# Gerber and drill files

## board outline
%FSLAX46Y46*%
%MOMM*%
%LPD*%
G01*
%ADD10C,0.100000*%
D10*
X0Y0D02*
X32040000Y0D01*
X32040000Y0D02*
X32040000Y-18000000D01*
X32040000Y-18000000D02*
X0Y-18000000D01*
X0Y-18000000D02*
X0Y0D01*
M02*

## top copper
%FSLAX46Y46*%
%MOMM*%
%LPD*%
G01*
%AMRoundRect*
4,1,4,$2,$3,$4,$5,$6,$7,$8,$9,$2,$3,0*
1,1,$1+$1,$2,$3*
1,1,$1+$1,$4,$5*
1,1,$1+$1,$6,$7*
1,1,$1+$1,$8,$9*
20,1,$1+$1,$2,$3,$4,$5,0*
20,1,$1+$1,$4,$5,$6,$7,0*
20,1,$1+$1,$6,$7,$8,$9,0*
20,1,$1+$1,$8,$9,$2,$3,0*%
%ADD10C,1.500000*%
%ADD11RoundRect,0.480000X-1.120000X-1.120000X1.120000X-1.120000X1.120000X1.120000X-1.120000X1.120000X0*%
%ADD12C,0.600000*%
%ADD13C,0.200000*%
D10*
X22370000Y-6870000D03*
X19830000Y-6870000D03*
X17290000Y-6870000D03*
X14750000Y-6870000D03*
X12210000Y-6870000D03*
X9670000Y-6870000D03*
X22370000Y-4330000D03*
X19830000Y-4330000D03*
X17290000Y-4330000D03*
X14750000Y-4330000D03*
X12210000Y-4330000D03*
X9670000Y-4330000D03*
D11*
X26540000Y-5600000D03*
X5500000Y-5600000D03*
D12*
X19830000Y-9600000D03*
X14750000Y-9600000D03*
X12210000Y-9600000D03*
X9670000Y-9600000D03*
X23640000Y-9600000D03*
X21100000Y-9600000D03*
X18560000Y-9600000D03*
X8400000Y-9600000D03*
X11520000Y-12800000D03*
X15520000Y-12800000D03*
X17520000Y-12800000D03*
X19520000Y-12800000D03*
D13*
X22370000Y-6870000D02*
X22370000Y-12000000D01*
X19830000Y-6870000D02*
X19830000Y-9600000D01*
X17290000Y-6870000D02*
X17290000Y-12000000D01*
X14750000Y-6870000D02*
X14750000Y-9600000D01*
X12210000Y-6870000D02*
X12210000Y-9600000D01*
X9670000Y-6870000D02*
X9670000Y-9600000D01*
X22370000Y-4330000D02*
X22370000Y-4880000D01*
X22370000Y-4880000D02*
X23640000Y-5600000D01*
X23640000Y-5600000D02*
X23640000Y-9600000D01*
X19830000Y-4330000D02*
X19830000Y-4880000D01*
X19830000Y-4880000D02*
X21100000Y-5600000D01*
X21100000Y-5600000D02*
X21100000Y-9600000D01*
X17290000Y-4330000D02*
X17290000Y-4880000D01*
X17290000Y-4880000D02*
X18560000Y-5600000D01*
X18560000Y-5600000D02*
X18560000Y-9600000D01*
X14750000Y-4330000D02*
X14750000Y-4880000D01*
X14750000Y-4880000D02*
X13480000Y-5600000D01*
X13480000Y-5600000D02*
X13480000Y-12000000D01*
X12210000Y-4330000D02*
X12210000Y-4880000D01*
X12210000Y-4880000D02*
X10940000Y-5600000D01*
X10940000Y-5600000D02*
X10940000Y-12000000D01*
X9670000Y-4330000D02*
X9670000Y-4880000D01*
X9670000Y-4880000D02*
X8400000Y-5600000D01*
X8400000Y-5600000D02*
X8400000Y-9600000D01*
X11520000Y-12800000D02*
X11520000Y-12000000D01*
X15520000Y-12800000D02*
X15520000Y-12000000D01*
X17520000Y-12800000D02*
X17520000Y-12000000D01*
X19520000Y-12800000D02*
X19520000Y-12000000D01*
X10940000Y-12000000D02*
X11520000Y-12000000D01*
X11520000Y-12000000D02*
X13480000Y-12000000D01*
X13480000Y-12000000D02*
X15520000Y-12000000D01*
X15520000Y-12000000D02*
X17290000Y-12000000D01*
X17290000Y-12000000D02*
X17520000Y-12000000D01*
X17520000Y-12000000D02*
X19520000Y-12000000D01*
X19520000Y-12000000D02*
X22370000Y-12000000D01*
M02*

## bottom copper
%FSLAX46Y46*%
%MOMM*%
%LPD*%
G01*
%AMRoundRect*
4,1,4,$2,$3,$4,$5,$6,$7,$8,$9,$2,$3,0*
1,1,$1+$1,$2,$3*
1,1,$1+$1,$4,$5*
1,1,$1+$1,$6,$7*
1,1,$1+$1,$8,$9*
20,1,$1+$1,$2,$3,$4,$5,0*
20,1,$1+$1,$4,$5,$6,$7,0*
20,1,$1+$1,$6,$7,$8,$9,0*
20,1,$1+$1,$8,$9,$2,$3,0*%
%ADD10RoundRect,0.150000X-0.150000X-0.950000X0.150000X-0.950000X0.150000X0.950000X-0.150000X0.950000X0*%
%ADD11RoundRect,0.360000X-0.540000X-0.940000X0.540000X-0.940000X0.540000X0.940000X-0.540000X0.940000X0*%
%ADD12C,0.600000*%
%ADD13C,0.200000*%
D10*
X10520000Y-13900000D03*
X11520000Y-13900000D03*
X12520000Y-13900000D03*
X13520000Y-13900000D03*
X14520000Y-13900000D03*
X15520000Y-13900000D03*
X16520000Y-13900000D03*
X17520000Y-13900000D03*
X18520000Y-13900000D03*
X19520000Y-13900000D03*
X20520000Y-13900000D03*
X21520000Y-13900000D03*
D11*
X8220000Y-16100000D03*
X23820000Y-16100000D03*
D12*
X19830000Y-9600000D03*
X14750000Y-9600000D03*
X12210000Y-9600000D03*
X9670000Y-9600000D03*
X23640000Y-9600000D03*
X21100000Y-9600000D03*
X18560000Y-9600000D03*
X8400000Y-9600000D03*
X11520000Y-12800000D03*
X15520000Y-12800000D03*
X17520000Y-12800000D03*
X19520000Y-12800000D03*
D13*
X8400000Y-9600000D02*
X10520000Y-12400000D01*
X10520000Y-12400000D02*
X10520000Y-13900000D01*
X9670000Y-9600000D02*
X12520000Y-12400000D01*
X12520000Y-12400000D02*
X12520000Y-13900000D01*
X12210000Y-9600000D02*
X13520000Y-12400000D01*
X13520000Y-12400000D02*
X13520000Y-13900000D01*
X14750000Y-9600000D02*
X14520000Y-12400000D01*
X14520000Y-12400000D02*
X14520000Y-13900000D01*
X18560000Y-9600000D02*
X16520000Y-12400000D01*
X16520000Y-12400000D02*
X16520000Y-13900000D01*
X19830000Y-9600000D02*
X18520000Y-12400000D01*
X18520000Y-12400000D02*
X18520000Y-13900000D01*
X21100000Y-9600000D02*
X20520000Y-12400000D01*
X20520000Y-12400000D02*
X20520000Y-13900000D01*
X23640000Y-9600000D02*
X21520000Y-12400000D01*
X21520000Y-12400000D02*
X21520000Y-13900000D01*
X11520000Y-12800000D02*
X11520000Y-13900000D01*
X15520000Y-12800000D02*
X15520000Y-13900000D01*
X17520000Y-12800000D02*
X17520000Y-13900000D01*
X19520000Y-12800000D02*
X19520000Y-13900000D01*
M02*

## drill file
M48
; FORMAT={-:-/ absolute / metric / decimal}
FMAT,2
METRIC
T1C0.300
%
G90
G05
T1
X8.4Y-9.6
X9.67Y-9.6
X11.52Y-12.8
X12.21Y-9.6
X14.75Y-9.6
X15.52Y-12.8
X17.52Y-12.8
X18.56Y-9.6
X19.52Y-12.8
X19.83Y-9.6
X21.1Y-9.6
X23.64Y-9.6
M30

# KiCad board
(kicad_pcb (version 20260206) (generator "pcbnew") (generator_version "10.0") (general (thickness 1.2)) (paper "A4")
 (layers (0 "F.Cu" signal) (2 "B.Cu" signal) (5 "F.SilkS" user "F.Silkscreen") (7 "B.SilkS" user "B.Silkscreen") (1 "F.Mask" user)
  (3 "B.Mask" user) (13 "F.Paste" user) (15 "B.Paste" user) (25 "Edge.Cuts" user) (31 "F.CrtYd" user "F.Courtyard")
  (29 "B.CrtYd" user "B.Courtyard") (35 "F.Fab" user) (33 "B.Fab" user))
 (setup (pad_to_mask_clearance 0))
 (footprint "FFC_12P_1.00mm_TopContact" (at 16.02 15) (layer "B.Cu")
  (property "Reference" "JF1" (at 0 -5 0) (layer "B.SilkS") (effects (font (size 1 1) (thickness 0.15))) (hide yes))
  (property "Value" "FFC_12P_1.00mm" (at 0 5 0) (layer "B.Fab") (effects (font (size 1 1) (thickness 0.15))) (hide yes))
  (pad "1" smd roundrect (at -5.500 -1.1) (size 0.6 2.2) (layers "B.Cu" "B.Mask" "B.Paste") (roundrect_rratio 0.25) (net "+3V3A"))
  (pad "2" smd roundrect (at -4.500 -1.1) (size 0.6 2.2) (layers "B.Cu" "B.Mask" "B.Paste") (roundrect_rratio 0.25) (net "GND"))
  (pad "3" smd roundrect (at -3.500 -1.1) (size 0.6 2.2) (layers "B.Cu" "B.Mask" "B.Paste") (roundrect_rratio 0.25) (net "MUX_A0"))
  (pad "4" smd roundrect (at -2.500 -1.1) (size 0.6 2.2) (layers "B.Cu" "B.Mask" "B.Paste") (roundrect_rratio 0.25) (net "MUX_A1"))
  (pad "5" smd roundrect (at -1.500 -1.1) (size 0.6 2.2) (layers "B.Cu" "B.Mask" "B.Paste") (roundrect_rratio 0.25) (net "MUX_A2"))
  (pad "6" smd roundrect (at -0.500 -1.1) (size 0.6 2.2) (layers "B.Cu" "B.Mask" "B.Paste") (roundrect_rratio 0.25) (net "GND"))
  (pad "7" smd roundrect (at 0.500 -1.1) (size 0.6 2.2) (layers "B.Cu" "B.Mask" "B.Paste") (roundrect_rratio 0.25) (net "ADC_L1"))
  (pad "8" smd roundrect (at 1.500 -1.1) (size 0.6 2.2) (layers "B.Cu" "B.Mask" "B.Paste") (roundrect_rratio 0.25) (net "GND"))
  (pad "9" smd roundrect (at 2.500 -1.1) (size 0.6 2.2) (layers "B.Cu" "B.Mask" "B.Paste") (roundrect_rratio 0.25) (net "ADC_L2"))
  (pad "10" smd roundrect (at 3.500 -1.1) (size 0.6 2.2) (layers "B.Cu" "B.Mask" "B.Paste") (roundrect_rratio 0.25) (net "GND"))
  (pad "11" smd roundrect (at 4.500 -1.1) (size 0.6 2.2) (layers "B.Cu" "B.Mask" "B.Paste") (roundrect_rratio 0.25) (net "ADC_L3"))
  (pad "12" smd roundrect (at 5.500 -1.1) (size 0.6 2.2) (layers "B.Cu" "B.Mask" "B.Paste") (roundrect_rratio 0.25) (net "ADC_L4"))
  (pad "MP" smd roundrect (at -7.800 1.1) (size 1.8 2.6) (layers "B.Cu" "B.Mask" "B.Paste") (roundrect_rratio 0.2))
  (pad "MP" smd roundrect (at 7.800 1.1) (size 1.8 2.6) (layers "B.Cu" "B.Mask" "B.Paste") (roundrect_rratio 0.2)))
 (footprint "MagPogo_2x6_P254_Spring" (at 16.02 5.6 180) (layer "F.Cu")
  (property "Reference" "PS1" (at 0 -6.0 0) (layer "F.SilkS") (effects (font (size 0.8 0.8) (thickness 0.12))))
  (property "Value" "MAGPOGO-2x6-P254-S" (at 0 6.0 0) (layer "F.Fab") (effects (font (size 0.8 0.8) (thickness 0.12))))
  (pad "1" smd circle (at -6.35 -1.27) (size 1.5 1.5) (layers "F.Cu" "F.Paste" "F.Mask") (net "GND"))
  (pad "2" smd circle (at -3.81 -1.27) (size 1.5 1.5) (layers "F.Cu" "F.Paste" "F.Mask") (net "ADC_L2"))
  (pad "3" smd circle (at -1.27 -1.27) (size 1.5 1.5) (layers "F.Cu" "F.Paste" "F.Mask") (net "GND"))
  (pad "4" smd circle (at 1.27 -1.27) (size 1.5 1.5) (layers "F.Cu" "F.Paste" "F.Mask") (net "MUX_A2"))
  (pad "5" smd circle (at 3.81 -1.27) (size 1.5 1.5) (layers "F.Cu" "F.Paste" "F.Mask") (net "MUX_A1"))
  (pad "6" smd circle (at 6.35 -1.27) (size 1.5 1.5) (layers "F.Cu" "F.Paste" "F.Mask") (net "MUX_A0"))
  (pad "7" smd circle (at -6.35 1.27) (size 1.5 1.5) (layers "F.Cu" "F.Paste" "F.Mask") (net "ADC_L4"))
  (pad "8" smd circle (at -3.81 1.27) (size 1.5 1.5) (layers "F.Cu" "F.Paste" "F.Mask") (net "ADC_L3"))
  (pad "9" smd circle (at -1.27 1.27) (size 1.5 1.5) (layers "F.Cu" "F.Paste" "F.Mask") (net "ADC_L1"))
  (pad "10" smd circle (at 1.27 1.27) (size 1.5 1.5) (layers "F.Cu" "F.Paste" "F.Mask") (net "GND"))
  (pad "11" smd circle (at 3.81 1.27) (size 1.5 1.5) (layers "F.Cu" "F.Paste" "F.Mask") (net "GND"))
  (pad "12" smd circle (at 6.35 1.27) (size 1.5 1.5) (layers "F.Cu" "F.Paste" "F.Mask") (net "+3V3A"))
  (pad "MP1" smd roundrect (at -10.52 0) (size 3.2 3.2) (roundrect_rratio 0.15) (layers "F.Cu" "F.Paste" "F.Mask"))
  (pad "MP2" smd roundrect (at 10.52 0) (size 3.2 3.2) (roundrect_rratio 0.15) (layers "F.Cu" "F.Paste" "F.Mask")))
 (gr_line (start 0 0) (end 32.04 0) (stroke (width 0.1) (type solid)) (layer "Edge.Cuts"))
 (gr_line (start 32.04 0) (end 32.04 18) (stroke (width 0.1) (type solid)) (layer "Edge.Cuts"))
 (gr_line (start 32.04 18) (end 0 18) (stroke (width 0.1) (type solid)) (layer "Edge.Cuts"))
 (gr_line (start 0 18) (end 0 0) (stroke (width 0.1) (type solid)) (layer "Edge.Cuts"))
 (segment (start 22.37 6.87) (end 22.37 12) (width 0.2) (layer "F.Cu") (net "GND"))
 (segment (start 19.83 6.87) (end 19.83 9.6) (width 0.2) (layer "F.Cu") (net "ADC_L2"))
 (via (at 19.83 9.6) (size 0.6) (drill 0.3) (layers "F.Cu" "B.Cu") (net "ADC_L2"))
 (segment (start 17.29 6.87) (end 17.29 12) (width 0.2) (layer "F.Cu") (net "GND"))
 (segment (start 14.75 6.87) (end 14.75 9.6) (width 0.2) (layer "F.Cu") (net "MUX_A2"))
 (via (at 14.75 9.6) (size 0.6) (drill 0.3) (layers "F.Cu" "B.Cu") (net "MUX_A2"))
 (segment (start 12.21 6.87) (end 12.21 9.6) (width 0.2) (layer "F.Cu") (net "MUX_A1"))
 (via (at 12.21 9.6) (size 0.6) (drill 0.3) (layers "F.Cu" "B.Cu") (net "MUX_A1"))
 (segment (start 9.67 6.87) (end 9.67 9.6) (width 0.2) (layer "F.Cu") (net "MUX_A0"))
 (via (at 9.67 9.6) (size 0.6) (drill 0.3) (layers "F.Cu" "B.Cu") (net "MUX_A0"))
 (segment (start 22.37 4.33) (end 22.37 4.88) (width 0.2) (layer "F.Cu") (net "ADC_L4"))
 (segment (start 22.37 4.88) (end 23.64 5.6) (width 0.2) (layer "F.Cu") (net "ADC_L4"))
 (segment (start 23.64 5.6) (end 23.64 9.6) (width 0.2) (layer "F.Cu") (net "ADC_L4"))
 (via (at 23.64 9.6) (size 0.6) (drill 0.3) (layers "F.Cu" "B.Cu") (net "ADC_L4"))
 (segment (start 19.83 4.33) (end 19.83 4.88) (width 0.2) (layer "F.Cu") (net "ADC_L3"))
 (segment (start 19.83 4.88) (end 21.1 5.6) (width 0.2) (layer "F.Cu") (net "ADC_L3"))
 (segment (start 21.1 5.6) (end 21.1 9.6) (width 0.2) (layer "F.Cu") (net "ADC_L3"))
 (via (at 21.1 9.6) (size 0.6) (drill 0.3) (layers "F.Cu" "B.Cu") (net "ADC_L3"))
 (segment (start 17.29 4.33) (end 17.29 4.88) (width 0.2) (layer "F.Cu") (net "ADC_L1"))
 (segment (start 17.29 4.88) (end 18.56 5.6) (width 0.2) (layer "F.Cu") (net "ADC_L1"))
 (segment (start 18.56 5.6) (end 18.56 9.6) (width 0.2) (layer "F.Cu") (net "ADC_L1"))
 (via (at 18.56 9.6) (size 0.6) (drill 0.3) (layers "F.Cu" "B.Cu") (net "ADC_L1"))
 (segment (start 14.75 4.33) (end 14.75 4.88) (width 0.2) (layer "F.Cu") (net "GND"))
 (segment (start 14.75 4.88) (end 13.48 5.6) (width 0.2) (layer "F.Cu") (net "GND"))
 (segment (start 13.48 5.6) (end 13.48 12) (width 0.2) (layer "F.Cu") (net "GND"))
 (segment (start 12.21 4.33) (end 12.21 4.88) (width 0.2) (layer "F.Cu") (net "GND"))
 (segment (start 12.21 4.88) (end 10.94 5.6) (width 0.2) (layer "F.Cu") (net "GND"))
 (segment (start 10.94 5.6) (end 10.94 12) (width 0.2) (layer "F.Cu") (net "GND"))
 (segment (start 9.67 4.33) (end 9.67 4.88) (width 0.2) (layer "F.Cu") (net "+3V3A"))
 (segment (start 9.67 4.88) (end 8.4 5.6) (width 0.2) (layer "F.Cu") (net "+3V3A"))
 (segment (start 8.4 5.6) (end 8.4 9.6) (width 0.2) (layer "F.Cu") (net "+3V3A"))
 (via (at 8.4 9.6) (size 0.6) (drill 0.3) (layers "F.Cu" "B.Cu") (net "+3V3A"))
 (segment (start 8.4 9.6) (end 10.52 12.4) (width 0.2) (layer "B.Cu") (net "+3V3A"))
 (segment (start 10.52 12.4) (end 10.52 13.9) (width 0.2) (layer "B.Cu") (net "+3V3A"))
 (segment (start 9.67 9.6) (end 12.52 12.4) (width 0.2) (layer "B.Cu") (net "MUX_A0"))
 (segment (start 12.52 12.4) (end 12.52 13.9) (width 0.2) (layer "B.Cu") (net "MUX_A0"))
 (segment (start 12.21 9.6) (end 13.52 12.4) (width 0.2) (layer "B.Cu") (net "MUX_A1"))
 (segment (start 13.52 12.4) (end 13.52 13.9) (width 0.2) (layer "B.Cu") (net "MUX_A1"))
 (segment (start 14.75 9.6) (end 14.52 12.4) (width 0.2) (layer "B.Cu") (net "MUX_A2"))
 (segment (start 14.52 12.4) (end 14.52 13.9) (width 0.2) (layer "B.Cu") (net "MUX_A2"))
 (segment (start 18.56 9.6) (end 16.52 12.4) (width 0.2) (layer "B.Cu") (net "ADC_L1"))
 (segment (start 16.52 12.4) (end 16.52 13.9) (width 0.2) (layer "B.Cu") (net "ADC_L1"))
 (segment (start 19.83 9.6) (end 18.52 12.4) (width 0.2) (layer "B.Cu") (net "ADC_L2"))
 (segment (start 18.52 12.4) (end 18.52 13.9) (width 0.2) (layer "B.Cu") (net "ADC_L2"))
 (segment (start 21.1 9.6) (end 20.52 12.4) (width 0.2) (layer "B.Cu") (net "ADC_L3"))
 (segment (start 20.52 12.4) (end 20.52 13.9) (width 0.2) (layer "B.Cu") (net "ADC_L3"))
 (segment (start 23.64 9.6) (end 21.52 12.4) (width 0.2) (layer "B.Cu") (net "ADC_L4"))
 (segment (start 21.52 12.4) (end 21.52 13.9) (width 0.2) (layer "B.Cu") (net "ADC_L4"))
 (segment (start 11.52 12.8) (end 11.52 13.9) (width 0.2) (layer "B.Cu") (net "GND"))
 (via (at 11.52 12.8) (size 0.6) (drill 0.3) (layers "F.Cu" "B.Cu") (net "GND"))
 (segment (start 11.52 12.8) (end 11.52 12) (width 0.2) (layer "F.Cu") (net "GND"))
 (segment (start 15.52 12.8) (end 15.52 13.9) (width 0.2) (layer "B.Cu") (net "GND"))
 (via (at 15.52 12.8) (size 0.6) (drill 0.3) (layers "F.Cu" "B.Cu") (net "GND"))
 (segment (start 15.52 12.8) (end 15.52 12) (width 0.2) (layer "F.Cu") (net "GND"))
 (segment (start 17.52 12.8) (end 17.52 13.9) (width 0.2) (layer "B.Cu") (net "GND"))
 (via (at 17.52 12.8) (size 0.6) (drill 0.3) (layers "F.Cu" "B.Cu") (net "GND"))
 (segment (start 17.52 12.8) (end 17.52 12) (width 0.2) (layer "F.Cu") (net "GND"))
 (segment (start 19.52 12.8) (end 19.52 13.9) (width 0.2) (layer "B.Cu") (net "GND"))
 (via (at 19.52 12.8) (size 0.6) (drill 0.3) (layers "F.Cu" "B.Cu") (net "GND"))
 (segment (start 19.52 12.8) (end 19.52 12) (width 0.2) (layer "F.Cu") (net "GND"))
 (segment (start 10.94 12) (end 11.52 12) (width 0.2) (layer "F.Cu") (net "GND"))
 (segment (start 11.52 12) (end 13.48 12) (width 0.2) (layer "F.Cu") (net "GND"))
 (segment (start 13.48 12) (end 15.52 12) (width 0.2) (layer "F.Cu") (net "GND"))
 (segment (start 15.52 12) (end 17.29 12) (width 0.2) (layer "F.Cu") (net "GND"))
 (segment (start 17.29 12) (end 17.52 12) (width 0.2) (layer "F.Cu") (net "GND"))
 (segment (start 17.52 12) (end 19.52 12) (width 0.2) (layer "F.Cu") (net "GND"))
 (segment (start 19.52 12) (end 22.37 12) (width 0.2) (layer "F.Cu") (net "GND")))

